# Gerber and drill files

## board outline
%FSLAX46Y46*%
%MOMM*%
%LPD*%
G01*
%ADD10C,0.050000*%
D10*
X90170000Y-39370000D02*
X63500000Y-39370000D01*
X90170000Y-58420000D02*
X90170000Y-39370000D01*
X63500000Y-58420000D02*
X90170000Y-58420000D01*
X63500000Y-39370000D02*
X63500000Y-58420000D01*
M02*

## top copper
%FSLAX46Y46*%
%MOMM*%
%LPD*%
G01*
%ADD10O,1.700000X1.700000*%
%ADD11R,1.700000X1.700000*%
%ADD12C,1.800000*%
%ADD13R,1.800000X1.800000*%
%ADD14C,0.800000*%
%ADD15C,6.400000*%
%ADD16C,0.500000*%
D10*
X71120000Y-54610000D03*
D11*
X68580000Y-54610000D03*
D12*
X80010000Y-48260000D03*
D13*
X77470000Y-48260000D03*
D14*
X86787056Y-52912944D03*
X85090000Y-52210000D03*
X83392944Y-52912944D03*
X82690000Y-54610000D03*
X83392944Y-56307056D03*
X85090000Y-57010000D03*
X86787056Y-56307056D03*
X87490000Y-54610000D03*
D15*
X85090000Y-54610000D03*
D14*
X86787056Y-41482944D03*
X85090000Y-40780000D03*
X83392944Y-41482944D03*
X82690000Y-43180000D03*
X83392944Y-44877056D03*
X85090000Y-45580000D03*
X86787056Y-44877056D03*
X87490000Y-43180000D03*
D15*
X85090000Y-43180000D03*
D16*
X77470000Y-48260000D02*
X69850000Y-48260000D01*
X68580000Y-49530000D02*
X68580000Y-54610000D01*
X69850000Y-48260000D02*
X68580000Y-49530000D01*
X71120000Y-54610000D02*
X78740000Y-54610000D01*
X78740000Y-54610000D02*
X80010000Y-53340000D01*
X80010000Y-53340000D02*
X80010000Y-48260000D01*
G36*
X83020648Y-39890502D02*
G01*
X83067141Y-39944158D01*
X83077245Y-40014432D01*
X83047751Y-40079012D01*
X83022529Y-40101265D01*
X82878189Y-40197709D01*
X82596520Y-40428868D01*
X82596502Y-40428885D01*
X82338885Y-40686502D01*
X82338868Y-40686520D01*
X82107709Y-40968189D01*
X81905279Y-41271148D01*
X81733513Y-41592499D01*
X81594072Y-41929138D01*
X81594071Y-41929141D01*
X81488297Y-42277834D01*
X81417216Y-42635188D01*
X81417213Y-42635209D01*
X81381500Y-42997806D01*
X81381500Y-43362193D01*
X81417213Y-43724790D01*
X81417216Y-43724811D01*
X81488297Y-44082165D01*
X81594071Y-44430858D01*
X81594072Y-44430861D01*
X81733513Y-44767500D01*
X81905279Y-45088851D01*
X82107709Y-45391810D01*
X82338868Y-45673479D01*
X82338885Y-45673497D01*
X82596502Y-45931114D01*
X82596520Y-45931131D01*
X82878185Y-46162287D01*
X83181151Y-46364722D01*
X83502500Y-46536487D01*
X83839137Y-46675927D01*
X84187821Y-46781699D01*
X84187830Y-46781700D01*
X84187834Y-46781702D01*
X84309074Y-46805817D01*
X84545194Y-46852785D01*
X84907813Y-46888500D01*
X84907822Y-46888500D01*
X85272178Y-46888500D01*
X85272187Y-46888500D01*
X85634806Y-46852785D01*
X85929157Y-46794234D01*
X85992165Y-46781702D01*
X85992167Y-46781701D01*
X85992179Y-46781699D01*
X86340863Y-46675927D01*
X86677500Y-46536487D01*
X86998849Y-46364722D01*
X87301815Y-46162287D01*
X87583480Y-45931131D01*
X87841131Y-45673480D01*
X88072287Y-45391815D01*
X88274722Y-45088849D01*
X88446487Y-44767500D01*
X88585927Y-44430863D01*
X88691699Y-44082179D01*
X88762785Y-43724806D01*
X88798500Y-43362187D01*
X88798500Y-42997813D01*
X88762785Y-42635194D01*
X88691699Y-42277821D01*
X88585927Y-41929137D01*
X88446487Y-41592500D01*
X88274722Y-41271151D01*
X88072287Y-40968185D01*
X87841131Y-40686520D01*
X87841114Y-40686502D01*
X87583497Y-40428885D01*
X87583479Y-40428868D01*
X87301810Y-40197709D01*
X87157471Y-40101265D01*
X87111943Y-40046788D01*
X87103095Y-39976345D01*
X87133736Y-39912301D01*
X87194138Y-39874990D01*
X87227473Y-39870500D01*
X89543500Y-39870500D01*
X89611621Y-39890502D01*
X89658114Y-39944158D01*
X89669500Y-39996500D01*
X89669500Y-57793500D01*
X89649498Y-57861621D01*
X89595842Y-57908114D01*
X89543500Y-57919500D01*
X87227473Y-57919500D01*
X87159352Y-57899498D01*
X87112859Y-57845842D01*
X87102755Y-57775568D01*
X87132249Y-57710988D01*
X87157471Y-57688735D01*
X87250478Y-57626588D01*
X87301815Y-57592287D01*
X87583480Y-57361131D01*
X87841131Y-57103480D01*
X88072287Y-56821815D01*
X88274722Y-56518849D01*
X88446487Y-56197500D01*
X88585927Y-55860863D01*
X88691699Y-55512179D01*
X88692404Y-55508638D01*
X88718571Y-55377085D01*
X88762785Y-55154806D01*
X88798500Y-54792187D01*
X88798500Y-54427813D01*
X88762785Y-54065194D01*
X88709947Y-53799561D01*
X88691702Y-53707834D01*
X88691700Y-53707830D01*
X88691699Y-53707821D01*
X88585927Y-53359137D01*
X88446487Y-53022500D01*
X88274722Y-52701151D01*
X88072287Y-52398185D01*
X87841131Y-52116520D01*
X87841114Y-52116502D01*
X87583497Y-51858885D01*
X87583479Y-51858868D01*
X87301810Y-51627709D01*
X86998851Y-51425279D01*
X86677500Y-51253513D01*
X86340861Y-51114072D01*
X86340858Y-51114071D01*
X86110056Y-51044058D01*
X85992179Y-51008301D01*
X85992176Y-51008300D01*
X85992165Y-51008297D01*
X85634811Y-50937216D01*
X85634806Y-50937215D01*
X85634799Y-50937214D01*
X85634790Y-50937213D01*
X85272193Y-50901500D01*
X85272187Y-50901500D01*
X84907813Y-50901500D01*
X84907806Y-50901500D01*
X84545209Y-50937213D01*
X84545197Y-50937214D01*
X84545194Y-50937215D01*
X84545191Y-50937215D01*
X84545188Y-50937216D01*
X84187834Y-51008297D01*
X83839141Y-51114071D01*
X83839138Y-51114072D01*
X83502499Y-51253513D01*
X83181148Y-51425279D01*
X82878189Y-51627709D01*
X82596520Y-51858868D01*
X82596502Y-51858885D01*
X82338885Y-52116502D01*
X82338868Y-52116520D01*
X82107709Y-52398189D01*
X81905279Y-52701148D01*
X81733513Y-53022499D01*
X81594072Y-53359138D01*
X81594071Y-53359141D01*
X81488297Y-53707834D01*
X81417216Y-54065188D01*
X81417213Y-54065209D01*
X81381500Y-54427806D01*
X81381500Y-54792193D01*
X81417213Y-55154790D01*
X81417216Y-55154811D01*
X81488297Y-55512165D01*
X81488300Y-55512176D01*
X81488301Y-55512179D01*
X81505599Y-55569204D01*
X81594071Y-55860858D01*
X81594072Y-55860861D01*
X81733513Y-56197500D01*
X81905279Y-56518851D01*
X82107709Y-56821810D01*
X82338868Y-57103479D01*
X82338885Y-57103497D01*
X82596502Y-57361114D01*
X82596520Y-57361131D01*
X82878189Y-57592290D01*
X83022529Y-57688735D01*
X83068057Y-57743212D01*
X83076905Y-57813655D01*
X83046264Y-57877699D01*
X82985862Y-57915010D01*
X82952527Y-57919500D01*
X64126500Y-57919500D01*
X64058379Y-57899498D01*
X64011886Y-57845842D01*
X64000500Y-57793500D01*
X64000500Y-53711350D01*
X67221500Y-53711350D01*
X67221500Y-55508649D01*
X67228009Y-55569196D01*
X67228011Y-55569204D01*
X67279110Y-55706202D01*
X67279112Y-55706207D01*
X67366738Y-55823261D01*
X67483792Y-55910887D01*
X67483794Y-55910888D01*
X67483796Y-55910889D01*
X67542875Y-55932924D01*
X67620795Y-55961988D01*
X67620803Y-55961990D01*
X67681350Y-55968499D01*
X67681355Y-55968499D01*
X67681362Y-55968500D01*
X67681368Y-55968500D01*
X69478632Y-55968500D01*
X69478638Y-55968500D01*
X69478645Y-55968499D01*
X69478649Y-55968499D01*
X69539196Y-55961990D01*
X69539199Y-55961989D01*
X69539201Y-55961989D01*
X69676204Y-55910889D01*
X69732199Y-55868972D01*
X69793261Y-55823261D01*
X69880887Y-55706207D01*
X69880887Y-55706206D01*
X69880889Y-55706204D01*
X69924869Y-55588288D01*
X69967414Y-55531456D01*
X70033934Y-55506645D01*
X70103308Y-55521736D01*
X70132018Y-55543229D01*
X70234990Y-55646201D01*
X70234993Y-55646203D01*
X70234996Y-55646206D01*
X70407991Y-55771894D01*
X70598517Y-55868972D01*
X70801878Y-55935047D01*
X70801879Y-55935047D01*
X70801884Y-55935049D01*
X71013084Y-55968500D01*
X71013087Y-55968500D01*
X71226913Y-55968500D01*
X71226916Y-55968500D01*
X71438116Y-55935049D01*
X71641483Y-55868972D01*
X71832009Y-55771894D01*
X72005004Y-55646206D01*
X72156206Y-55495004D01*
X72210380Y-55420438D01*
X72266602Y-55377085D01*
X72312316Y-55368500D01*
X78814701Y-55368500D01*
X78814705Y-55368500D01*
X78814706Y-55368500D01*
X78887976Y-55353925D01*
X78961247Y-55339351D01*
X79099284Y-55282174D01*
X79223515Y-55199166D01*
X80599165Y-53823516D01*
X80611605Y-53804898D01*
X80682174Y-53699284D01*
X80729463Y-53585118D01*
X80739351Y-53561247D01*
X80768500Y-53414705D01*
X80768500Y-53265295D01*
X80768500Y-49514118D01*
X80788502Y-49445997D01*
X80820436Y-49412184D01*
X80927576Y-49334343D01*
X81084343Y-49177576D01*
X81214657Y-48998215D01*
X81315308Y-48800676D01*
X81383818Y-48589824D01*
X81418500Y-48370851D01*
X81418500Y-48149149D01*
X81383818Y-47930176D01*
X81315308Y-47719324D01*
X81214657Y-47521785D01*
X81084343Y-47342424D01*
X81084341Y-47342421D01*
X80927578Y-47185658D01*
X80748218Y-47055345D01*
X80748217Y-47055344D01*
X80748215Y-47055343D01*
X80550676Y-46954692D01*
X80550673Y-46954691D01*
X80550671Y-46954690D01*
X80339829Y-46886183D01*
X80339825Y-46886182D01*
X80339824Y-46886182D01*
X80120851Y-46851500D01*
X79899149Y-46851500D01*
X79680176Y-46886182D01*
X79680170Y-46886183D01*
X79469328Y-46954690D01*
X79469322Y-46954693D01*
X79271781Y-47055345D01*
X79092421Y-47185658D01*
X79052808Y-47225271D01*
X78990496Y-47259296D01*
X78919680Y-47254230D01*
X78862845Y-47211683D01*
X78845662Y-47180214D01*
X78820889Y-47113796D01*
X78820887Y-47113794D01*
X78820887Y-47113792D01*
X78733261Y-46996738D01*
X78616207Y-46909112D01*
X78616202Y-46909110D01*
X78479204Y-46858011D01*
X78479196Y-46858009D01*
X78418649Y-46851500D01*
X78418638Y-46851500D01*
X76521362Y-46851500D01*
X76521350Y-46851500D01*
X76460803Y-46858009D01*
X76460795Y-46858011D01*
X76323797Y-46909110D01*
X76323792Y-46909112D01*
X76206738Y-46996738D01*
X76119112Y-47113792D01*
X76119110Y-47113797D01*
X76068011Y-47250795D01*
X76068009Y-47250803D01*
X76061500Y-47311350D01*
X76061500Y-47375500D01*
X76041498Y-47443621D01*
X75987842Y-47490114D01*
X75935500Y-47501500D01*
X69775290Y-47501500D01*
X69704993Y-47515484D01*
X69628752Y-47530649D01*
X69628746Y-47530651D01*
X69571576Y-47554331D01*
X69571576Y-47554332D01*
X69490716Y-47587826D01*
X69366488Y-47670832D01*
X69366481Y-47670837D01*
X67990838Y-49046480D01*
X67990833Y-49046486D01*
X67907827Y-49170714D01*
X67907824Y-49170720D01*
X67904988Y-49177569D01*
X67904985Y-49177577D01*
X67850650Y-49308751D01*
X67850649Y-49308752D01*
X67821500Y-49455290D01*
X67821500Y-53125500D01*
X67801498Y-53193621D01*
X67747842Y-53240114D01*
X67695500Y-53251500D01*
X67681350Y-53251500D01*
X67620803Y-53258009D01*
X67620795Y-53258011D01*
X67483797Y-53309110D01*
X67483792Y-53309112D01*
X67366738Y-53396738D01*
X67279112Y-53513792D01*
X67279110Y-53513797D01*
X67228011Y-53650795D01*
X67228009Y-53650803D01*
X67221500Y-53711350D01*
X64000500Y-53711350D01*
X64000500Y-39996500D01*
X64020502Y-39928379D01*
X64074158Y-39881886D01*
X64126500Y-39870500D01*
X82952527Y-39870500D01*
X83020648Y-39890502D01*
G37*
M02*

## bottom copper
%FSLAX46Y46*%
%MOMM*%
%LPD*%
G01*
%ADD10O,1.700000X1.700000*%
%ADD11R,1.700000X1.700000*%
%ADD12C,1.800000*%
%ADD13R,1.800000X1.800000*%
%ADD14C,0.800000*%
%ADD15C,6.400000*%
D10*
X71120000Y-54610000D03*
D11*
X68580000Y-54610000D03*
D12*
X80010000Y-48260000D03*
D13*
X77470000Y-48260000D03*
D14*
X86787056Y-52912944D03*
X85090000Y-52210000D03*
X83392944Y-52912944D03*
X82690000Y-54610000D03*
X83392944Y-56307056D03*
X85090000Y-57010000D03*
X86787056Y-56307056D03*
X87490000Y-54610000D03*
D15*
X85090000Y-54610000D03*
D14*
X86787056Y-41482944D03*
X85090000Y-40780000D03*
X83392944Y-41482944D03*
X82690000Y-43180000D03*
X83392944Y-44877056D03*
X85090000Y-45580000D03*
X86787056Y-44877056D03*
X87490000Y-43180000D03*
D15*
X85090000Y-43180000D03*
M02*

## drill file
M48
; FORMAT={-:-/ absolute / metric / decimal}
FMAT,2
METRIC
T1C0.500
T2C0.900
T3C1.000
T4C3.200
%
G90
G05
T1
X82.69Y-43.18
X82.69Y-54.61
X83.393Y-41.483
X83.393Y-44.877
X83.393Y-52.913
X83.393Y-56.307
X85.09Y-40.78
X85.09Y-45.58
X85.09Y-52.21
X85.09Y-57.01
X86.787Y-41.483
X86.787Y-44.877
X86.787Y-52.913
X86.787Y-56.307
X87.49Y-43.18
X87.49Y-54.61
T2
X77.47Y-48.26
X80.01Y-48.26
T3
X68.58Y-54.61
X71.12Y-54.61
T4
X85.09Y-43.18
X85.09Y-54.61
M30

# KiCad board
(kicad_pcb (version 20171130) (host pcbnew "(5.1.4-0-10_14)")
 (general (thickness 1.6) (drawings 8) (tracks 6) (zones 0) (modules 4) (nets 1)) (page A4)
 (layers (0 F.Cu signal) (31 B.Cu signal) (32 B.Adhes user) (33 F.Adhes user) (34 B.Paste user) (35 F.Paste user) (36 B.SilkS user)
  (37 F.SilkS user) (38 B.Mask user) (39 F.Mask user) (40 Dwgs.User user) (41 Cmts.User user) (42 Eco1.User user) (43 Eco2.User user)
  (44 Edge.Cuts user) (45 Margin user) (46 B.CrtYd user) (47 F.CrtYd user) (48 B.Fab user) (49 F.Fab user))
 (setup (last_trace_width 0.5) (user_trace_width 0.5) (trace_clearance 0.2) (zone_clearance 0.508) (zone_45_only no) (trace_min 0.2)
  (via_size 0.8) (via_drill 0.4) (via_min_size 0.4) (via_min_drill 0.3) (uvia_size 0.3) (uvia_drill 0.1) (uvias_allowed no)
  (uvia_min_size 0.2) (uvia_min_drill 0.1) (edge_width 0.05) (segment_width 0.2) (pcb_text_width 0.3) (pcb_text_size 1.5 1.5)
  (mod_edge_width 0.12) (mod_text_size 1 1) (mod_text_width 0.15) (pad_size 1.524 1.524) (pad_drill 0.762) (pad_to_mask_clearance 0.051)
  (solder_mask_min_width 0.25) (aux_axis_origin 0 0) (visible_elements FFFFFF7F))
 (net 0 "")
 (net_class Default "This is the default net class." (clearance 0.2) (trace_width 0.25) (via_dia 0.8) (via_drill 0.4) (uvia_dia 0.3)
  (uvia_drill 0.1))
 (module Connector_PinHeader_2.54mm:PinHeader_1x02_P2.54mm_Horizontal (layer F.Cu) (at 68.58 54.61 90)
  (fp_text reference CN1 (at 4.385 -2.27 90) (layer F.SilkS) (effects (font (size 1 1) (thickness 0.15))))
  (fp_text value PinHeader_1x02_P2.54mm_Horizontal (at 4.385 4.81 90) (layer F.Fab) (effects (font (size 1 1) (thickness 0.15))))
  (pad 2 thru_hole oval (at 0 2.54 90) (size 1.7 1.7) (drill 1) (layers *.Cu *.Mask))
  (pad 1 thru_hole rect (at 0 0 90) (size 1.7 1.7) (drill 1) (layers *.Cu *.Mask)))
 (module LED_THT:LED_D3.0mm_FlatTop (layer F.Cu) (at 77.47 48.26)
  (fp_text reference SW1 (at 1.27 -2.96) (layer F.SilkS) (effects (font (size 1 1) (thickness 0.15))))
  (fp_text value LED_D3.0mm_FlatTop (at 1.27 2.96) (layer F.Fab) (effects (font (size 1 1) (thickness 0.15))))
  (pad 2 thru_hole circle (at 2.54 0) (size 1.8 1.8) (drill 0.9) (layers *.Cu *.Mask))
  (pad 1 thru_hole rect (at 0 0) (size 1.8 1.8) (drill 0.9) (layers *.Cu *.Mask)))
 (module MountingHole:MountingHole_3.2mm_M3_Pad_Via (layer F.Cu) (at 85.09 54.61)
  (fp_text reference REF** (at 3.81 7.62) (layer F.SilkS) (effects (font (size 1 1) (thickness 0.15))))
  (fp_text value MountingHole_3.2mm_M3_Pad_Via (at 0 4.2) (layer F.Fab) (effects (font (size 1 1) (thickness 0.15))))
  (pad 1 thru_hole circle (at 1.697056 -1.697056) (size 0.8 0.8) (drill 0.5) (layers *.Cu *.Mask))
  (pad 1 thru_hole circle (at 0 -2.4) (size 0.8 0.8) (drill 0.5) (layers *.Cu *.Mask))
  (pad 1 thru_hole circle (at -1.697056 -1.697056) (size 0.8 0.8) (drill 0.5) (layers *.Cu *.Mask))
  (pad 1 thru_hole circle (at -2.4 0) (size 0.8 0.8) (drill 0.5) (layers *.Cu *.Mask))
  (pad 1 thru_hole circle (at -1.697056 1.697056) (size 0.8 0.8) (drill 0.5) (layers *.Cu *.Mask))
  (pad 1 thru_hole circle (at 0 2.4) (size 0.8 0.8) (drill 0.5) (layers *.Cu *.Mask))
  (pad 1 thru_hole circle (at 1.697056 1.697056) (size 0.8 0.8) (drill 0.5) (layers *.Cu *.Mask))
  (pad 1 thru_hole circle (at 2.4 0) (size 0.8 0.8) (drill 0.5) (layers *.Cu *.Mask))
  (pad 1 thru_hole circle (at 0 0) (size 6.4 6.4) (drill 3.2) (layers *.Cu *.Mask)))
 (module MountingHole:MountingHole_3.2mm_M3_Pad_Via (layer F.Cu) (at 85.09 43.18)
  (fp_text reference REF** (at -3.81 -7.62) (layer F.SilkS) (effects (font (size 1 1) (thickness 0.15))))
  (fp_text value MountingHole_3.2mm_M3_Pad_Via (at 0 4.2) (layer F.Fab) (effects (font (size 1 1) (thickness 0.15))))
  (pad 1 thru_hole circle (at 1.697056 -1.697056) (size 0.8 0.8) (drill 0.5) (layers *.Cu *.Mask))
  (pad 1 thru_hole circle (at 0 -2.4) (size 0.8 0.8) (drill 0.5) (layers *.Cu *.Mask))
  (pad 1 thru_hole circle (at -1.697056 -1.697056) (size 0.8 0.8) (drill 0.5) (layers *.Cu *.Mask))
  (pad 1 thru_hole circle (at -2.4 0) (size 0.8 0.8) (drill 0.5) (layers *.Cu *.Mask))
  (pad 1 thru_hole circle (at -1.697056 1.697056) (size 0.8 0.8) (drill 0.5) (layers *.Cu *.Mask))
  (pad 1 thru_hole circle (at 0 2.4) (size 0.8 0.8) (drill 0.5) (layers *.Cu *.Mask))
  (pad 1 thru_hole circle (at 1.697056 1.697056) (size 0.8 0.8) (drill 0.5) (layers *.Cu *.Mask))
  (pad 1 thru_hole circle (at 2.4 0) (size 0.8 0.8) (drill 0.5) (layers *.Cu *.Mask))
  (pad 1 thru_hole circle (at 0 0) (size 6.4 6.4) (drill 3.2) (layers *.Cu *.Mask)))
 (gr_line (start 90.17 39.37) (end 63.5 39.37) (layer Edge.Cuts) (width 0.05))
 (gr_line (start 90.17 58.42) (end 90.17 39.37) (layer Edge.Cuts) (width 0.05))
 (gr_line (start 63.5 58.42) (end 90.17 58.42) (layer Edge.Cuts) (width 0.05))
 (gr_line (start 63.5 39.37) (end 63.5 58.42) (layer Edge.Cuts) (width 0.05))
 (segment (start 77.47 48.26) (end 69.85 48.26) (width 0.5) (layer F.Cu) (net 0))
 (segment (start 68.58 49.53) (end 68.58 54.61) (width 0.5) (layer F.Cu) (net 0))
 (segment (start 69.85 48.26) (end 68.58 49.53) (width 0.5) (layer F.Cu) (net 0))
 (segment (start 71.12 54.61) (end 78.74 54.61) (width 0.5) (layer F.Cu) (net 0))
 (segment (start 78.74 54.61) (end 80.01 53.34) (width 0.5) (layer F.Cu) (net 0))
 (segment (start 80.01 53.34) (end 80.01 48.26) (width 0.5) (layer F.Cu) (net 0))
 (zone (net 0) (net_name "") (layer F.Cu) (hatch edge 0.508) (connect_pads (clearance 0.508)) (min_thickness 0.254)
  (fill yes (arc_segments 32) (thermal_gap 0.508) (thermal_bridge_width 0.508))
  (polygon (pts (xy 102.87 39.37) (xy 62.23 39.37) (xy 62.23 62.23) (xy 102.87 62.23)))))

